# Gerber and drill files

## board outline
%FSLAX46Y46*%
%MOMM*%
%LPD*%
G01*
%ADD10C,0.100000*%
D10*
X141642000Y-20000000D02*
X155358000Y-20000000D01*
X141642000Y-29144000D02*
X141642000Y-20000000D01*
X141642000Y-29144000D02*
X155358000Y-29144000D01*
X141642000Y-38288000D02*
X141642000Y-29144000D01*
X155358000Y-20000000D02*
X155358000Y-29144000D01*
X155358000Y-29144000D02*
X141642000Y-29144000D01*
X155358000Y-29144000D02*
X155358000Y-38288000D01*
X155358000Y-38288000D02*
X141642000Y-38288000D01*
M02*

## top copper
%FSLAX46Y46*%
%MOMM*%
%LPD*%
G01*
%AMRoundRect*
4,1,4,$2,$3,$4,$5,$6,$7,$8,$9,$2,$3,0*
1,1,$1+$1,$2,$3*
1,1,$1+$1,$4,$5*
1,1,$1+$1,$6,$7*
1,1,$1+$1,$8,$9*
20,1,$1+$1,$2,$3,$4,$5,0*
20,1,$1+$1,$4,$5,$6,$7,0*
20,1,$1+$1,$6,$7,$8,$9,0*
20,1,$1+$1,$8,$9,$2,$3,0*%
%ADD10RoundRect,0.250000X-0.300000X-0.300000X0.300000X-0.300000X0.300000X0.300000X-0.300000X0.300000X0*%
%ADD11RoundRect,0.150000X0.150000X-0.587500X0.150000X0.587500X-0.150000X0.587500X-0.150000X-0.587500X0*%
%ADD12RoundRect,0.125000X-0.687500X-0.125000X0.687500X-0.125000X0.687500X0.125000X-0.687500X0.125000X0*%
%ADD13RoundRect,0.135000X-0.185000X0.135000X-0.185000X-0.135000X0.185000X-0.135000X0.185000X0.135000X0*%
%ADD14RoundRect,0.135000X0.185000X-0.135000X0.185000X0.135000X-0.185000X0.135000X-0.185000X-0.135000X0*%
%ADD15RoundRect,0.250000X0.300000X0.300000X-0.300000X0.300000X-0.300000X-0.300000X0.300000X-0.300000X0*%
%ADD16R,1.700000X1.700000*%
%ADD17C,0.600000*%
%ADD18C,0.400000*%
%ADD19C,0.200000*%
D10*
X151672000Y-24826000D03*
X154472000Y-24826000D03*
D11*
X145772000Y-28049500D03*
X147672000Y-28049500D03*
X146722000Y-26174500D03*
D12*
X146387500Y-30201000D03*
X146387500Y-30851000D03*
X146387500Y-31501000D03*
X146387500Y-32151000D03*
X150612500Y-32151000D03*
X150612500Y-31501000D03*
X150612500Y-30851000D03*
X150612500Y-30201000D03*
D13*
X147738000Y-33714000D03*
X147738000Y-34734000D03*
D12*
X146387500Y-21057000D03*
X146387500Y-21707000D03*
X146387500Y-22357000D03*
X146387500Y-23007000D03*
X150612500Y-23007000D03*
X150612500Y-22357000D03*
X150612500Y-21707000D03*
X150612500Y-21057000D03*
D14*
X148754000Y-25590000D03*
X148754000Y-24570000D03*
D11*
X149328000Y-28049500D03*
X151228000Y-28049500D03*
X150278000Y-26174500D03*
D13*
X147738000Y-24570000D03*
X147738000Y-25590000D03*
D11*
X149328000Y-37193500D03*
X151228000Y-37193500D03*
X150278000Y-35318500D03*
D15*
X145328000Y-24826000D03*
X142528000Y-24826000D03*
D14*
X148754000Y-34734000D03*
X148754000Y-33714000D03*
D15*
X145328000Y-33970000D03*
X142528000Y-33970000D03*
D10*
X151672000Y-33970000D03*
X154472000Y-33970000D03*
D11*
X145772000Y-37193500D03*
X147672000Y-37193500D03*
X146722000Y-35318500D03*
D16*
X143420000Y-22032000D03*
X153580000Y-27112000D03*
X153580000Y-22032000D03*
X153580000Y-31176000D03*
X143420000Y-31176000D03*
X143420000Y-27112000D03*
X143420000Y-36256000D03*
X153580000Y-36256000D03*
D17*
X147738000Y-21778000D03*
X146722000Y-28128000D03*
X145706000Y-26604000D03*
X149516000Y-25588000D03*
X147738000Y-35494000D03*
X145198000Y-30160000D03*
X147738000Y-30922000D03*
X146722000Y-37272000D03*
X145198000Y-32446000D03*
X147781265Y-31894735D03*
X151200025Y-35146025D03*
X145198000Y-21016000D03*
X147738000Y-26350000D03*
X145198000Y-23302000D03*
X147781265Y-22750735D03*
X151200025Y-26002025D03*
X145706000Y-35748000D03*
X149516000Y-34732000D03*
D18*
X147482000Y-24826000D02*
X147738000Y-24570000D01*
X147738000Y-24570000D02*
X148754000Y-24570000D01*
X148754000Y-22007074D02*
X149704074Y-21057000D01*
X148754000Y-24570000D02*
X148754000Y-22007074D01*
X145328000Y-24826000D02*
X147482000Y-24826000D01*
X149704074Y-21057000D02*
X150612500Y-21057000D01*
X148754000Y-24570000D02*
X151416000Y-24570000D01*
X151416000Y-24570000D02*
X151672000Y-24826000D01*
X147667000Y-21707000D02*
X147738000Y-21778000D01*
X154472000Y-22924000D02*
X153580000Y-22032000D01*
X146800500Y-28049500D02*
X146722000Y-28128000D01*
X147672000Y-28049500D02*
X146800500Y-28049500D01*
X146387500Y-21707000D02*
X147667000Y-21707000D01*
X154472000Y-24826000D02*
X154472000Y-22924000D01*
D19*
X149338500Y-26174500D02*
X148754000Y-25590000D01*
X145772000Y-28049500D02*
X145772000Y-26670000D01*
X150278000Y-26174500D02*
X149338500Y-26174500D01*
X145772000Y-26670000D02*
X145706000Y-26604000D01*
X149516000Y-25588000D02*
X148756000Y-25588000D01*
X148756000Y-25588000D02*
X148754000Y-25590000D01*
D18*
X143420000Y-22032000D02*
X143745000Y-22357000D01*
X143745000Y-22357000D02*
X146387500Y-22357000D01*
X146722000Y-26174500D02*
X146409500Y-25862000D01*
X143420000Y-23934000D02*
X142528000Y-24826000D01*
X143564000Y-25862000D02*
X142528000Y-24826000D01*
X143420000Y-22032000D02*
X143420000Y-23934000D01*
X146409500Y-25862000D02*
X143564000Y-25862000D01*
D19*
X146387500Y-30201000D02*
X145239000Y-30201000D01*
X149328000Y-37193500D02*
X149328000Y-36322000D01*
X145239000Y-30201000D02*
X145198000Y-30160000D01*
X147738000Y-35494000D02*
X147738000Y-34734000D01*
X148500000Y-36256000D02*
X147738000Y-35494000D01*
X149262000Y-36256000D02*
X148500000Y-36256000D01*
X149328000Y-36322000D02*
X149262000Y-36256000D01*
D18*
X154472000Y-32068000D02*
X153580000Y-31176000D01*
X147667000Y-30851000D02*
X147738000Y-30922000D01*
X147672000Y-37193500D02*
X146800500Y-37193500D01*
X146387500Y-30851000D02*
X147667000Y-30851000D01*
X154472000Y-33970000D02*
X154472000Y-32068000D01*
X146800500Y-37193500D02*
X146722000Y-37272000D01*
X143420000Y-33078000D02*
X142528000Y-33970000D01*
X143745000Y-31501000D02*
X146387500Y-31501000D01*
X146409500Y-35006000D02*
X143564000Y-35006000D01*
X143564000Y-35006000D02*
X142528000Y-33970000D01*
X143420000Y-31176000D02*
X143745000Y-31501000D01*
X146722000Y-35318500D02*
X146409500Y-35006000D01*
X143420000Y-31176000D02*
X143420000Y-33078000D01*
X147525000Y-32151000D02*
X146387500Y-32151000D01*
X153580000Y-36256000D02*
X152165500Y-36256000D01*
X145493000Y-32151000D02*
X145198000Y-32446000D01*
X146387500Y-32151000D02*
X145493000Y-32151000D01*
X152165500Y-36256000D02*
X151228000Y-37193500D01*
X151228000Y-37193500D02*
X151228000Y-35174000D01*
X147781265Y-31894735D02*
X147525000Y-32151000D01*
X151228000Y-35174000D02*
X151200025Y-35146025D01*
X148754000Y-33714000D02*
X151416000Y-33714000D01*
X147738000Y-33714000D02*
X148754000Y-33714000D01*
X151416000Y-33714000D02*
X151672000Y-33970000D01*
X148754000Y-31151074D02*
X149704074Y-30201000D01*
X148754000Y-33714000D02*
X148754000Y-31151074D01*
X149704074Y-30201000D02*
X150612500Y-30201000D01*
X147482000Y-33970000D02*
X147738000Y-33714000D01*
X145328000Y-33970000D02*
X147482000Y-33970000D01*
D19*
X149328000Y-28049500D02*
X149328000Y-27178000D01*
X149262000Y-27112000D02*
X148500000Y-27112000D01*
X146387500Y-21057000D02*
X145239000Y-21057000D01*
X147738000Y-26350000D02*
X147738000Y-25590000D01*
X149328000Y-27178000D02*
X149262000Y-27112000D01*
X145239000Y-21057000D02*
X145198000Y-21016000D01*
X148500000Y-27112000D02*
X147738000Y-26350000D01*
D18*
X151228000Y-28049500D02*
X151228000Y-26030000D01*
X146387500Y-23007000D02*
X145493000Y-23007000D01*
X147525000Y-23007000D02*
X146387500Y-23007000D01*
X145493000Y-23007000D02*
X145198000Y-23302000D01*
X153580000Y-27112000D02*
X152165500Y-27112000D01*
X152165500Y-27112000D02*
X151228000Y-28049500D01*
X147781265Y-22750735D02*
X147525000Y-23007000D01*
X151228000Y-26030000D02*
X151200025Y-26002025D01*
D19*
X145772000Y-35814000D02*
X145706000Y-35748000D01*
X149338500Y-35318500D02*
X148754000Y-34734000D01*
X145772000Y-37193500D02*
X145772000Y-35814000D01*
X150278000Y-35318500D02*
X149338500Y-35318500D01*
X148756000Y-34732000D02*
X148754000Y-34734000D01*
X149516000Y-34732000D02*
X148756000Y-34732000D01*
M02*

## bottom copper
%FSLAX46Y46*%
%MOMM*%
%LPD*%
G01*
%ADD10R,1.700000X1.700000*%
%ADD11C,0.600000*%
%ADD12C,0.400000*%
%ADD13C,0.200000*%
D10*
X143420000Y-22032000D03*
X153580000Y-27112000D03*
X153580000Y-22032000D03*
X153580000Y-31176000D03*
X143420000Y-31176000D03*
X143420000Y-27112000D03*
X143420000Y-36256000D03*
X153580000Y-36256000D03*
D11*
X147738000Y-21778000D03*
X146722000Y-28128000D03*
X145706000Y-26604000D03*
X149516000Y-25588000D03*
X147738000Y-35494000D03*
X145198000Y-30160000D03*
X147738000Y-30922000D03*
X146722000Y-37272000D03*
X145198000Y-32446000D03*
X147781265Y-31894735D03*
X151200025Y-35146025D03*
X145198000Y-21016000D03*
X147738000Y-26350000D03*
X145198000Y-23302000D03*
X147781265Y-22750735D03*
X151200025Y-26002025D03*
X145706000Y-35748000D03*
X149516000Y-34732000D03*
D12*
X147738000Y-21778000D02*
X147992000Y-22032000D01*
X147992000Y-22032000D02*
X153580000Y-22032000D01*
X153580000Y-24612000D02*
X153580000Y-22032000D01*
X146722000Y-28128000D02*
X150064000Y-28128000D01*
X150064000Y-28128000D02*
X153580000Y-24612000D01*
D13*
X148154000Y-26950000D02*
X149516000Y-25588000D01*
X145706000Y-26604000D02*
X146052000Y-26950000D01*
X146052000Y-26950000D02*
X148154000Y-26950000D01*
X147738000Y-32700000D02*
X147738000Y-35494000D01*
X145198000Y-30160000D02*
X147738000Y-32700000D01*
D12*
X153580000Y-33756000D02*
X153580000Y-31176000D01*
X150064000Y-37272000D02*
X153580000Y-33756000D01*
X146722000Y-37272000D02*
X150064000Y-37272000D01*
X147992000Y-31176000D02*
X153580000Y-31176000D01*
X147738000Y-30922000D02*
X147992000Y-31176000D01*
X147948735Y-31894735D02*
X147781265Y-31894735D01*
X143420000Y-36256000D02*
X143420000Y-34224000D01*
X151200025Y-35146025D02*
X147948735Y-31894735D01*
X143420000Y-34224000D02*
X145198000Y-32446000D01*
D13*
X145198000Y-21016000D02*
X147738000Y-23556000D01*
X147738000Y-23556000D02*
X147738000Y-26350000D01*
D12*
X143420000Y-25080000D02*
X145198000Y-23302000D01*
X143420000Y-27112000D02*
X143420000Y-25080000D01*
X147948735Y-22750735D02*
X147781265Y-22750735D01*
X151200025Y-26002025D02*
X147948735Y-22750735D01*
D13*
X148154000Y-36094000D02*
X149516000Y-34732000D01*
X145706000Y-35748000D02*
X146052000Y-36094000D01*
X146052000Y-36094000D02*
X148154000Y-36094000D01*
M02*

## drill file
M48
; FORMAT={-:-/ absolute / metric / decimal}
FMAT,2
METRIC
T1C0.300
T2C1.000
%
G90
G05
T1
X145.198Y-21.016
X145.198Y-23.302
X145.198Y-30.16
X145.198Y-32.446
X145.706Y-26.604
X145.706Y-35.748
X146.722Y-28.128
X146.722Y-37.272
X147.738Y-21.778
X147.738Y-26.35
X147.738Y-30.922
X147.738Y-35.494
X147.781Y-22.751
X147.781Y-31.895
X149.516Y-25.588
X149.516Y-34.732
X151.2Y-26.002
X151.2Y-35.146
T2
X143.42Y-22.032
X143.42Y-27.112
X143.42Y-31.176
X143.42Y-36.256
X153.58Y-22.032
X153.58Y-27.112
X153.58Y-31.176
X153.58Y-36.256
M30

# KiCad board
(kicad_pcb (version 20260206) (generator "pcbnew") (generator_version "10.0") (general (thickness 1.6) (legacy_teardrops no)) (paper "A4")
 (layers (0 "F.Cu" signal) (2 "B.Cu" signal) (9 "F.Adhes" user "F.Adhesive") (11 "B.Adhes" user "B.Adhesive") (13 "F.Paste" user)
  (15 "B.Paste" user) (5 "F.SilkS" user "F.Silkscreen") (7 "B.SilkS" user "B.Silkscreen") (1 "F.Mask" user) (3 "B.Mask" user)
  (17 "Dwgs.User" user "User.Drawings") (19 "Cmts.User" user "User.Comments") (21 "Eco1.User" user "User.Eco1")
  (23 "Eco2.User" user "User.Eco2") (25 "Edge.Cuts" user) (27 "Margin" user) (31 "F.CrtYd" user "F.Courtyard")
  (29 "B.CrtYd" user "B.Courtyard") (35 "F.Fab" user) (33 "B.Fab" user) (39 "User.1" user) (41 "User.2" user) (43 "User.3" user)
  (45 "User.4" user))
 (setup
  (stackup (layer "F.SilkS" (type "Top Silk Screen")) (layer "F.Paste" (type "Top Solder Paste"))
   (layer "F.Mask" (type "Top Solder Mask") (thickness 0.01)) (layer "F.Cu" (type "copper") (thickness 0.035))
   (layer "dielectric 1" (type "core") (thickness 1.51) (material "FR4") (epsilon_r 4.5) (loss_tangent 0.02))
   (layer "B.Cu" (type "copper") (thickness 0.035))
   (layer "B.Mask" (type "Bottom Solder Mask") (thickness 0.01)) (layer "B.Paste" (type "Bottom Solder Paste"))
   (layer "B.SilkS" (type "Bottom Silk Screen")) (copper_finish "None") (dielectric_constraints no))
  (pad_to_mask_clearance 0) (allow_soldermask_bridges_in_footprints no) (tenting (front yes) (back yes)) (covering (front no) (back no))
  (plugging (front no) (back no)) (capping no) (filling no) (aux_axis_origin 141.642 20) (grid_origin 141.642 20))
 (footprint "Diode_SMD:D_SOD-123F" (layer "F.Cu") (at 153.072 24.826)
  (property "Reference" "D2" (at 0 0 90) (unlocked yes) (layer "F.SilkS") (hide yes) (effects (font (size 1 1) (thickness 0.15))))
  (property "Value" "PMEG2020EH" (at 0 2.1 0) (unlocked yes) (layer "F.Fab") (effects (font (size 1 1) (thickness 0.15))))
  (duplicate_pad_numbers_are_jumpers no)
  (pad "1" smd roundrect (at -1.4 0) (size 1.1 1.1) (layers "F.Cu" "F.Mask" "F.Paste") (roundrect_rratio 0.2272727273) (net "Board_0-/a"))
  (pad "2" smd roundrect (at 1.4 0) (size 1.1 1.1) (layers "F.Cu" "F.Mask" "F.Paste") (roundrect_rratio 0.2272727273) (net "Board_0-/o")))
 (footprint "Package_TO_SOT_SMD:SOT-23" (layer "F.Cu") (at 146.722 27.112 90)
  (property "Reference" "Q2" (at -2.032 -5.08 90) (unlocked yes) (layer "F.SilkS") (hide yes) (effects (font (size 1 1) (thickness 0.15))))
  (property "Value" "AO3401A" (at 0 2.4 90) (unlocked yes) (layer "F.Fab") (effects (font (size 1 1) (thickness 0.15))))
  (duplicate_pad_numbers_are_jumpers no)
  (pad "1" smd roundrect (at -0.9375 -0.95 90) (size 1.475 0.6) (layers "F.Cu" "F.Mask" "F.Paste") (roundrect_rratio 0.25)
   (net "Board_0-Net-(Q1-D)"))
  (pad "2" smd roundrect (at -0.9375 0.95 90) (size 1.475 0.6) (layers "F.Cu" "F.Mask" "F.Paste") (roundrect_rratio 0.25) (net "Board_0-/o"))
  (pad "3" smd roundrect (at 0.9375 0 90) (size 1.475 0.6) (layers "F.Cu" "F.Mask" "F.Paste") (roundrect_rratio 0.25) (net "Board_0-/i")))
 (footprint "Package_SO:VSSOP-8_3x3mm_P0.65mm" (layer "F.Cu") (at 148.5 31.176)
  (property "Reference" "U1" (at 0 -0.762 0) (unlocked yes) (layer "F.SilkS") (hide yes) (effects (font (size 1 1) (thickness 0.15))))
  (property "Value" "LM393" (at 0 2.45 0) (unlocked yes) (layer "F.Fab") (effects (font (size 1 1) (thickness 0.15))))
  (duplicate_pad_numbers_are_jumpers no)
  (pad "1" smd roundrect (at -2.1125 -0.975) (size 1.625 0.5) (layers "F.Cu" "F.Mask" "F.Paste") (roundrect_rratio 0.25)
   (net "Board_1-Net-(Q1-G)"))
  (pad "2" smd roundrect (at -2.1125 -0.325) (size 1.625 0.5) (layers "F.Cu" "F.Mask" "F.Paste") (roundrect_rratio 0.25) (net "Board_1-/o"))
  (pad "3" smd roundrect (at -2.1125 0.325) (size 1.625 0.5) (layers "F.Cu" "F.Mask" "F.Paste") (roundrect_rratio 0.25) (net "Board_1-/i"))
  (pad "4" smd roundrect (at -2.1125 0.975) (size 1.625 0.5) (layers "F.Cu" "F.Mask" "F.Paste") (roundrect_rratio 0.25) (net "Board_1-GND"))
  (pad "5" smd roundrect (at 2.1125 0.975) (size 1.625 0.5) (layers "F.Cu" "F.Mask" "F.Paste") (roundrect_rratio 0.25)
   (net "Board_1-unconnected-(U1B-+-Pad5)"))
  (pad "6" smd roundrect (at 2.1125 0.325) (size 1.625 0.5) (layers "F.Cu" "F.Mask" "F.Paste") (roundrect_rratio 0.25)
   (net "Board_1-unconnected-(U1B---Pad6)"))
  (pad "7" smd roundrect (at 2.1125 -0.325) (size 1.625 0.5) (layers "F.Cu" "F.Mask" "F.Paste") (roundrect_rratio 0.25)
   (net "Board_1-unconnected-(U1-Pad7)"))
  (pad "8" smd roundrect (at 2.1125 -0.975) (size 1.625 0.5) (layers "F.Cu" "F.Mask" "F.Paste") (roundrect_rratio 0.25) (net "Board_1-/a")))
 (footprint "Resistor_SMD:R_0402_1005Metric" (layer "F.Cu") (at 147.738 34.224 -90)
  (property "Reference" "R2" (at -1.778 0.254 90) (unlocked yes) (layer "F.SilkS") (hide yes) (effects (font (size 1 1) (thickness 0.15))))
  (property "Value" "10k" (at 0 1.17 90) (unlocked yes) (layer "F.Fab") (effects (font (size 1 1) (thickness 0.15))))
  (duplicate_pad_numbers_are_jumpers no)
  (pad "1" smd roundrect (at -0.51 0 270) (size 0.54 0.64) (layers "F.Cu" "F.Mask" "F.Paste") (roundrect_rratio 0.25) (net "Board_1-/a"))
  (pad "2" smd roundrect (at 0.51 0 270) (size 0.54 0.64) (layers "F.Cu" "F.Mask" "F.Paste") (roundrect_rratio 0.25)
   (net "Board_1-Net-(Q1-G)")))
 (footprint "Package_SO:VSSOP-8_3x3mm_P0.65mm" (layer "F.Cu") (at 148.5 22.032)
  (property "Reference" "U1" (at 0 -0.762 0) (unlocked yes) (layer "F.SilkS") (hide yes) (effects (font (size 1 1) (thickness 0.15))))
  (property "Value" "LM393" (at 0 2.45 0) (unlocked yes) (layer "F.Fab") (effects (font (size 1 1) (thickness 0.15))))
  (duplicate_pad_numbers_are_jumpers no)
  (pad "1" smd roundrect (at -2.1125 -0.975) (size 1.625 0.5) (layers "F.Cu" "F.Mask" "F.Paste") (roundrect_rratio 0.25)
   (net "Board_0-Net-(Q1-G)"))
  (pad "2" smd roundrect (at -2.1125 -0.325) (size 1.625 0.5) (layers "F.Cu" "F.Mask" "F.Paste") (roundrect_rratio 0.25) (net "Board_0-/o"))
  (pad "3" smd roundrect (at -2.1125 0.325) (size 1.625 0.5) (layers "F.Cu" "F.Mask" "F.Paste") (roundrect_rratio 0.25) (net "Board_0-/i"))
  (pad "4" smd roundrect (at -2.1125 0.975) (size 1.625 0.5) (layers "F.Cu" "F.Mask" "F.Paste") (roundrect_rratio 0.25) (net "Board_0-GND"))
  (pad "5" smd roundrect (at 2.1125 0.975) (size 1.625 0.5) (layers "F.Cu" "F.Mask" "F.Paste") (roundrect_rratio 0.25)
   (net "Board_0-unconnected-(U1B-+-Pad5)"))
  (pad "6" smd roundrect (at 2.1125 0.325) (size 1.625 0.5) (layers "F.Cu" "F.Mask" "F.Paste") (roundrect_rratio 0.25)
   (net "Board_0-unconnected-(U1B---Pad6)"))
  (pad "7" smd roundrect (at 2.1125 -0.325) (size 1.625 0.5) (layers "F.Cu" "F.Mask" "F.Paste") (roundrect_rratio 0.25)
   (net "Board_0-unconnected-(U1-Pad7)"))
  (pad "8" smd roundrect (at 2.1125 -0.975) (size 1.625 0.5) (layers "F.Cu" "F.Mask" "F.Paste") (roundrect_rratio 0.25) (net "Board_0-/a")))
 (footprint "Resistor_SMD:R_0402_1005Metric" (layer "F.Cu") (at 148.754 25.08 90)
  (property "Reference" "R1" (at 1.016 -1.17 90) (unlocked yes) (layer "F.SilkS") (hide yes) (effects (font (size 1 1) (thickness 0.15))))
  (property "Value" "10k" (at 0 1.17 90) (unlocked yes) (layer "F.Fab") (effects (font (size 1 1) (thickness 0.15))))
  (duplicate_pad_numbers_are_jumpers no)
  (pad "1" smd roundrect (at -0.51 0 90) (size 0.54 0.64) (layers "F.Cu" "F.Mask" "F.Paste") (roundrect_rratio 0.25)
   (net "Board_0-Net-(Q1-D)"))
  (pad "2" smd roundrect (at 0.51 0 90) (size 0.54 0.64) (layers "F.Cu" "F.Mask" "F.Paste") (roundrect_rratio 0.25) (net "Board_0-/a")))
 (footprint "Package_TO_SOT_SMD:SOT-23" (layer "F.Cu") (at 150.278 27.112 90)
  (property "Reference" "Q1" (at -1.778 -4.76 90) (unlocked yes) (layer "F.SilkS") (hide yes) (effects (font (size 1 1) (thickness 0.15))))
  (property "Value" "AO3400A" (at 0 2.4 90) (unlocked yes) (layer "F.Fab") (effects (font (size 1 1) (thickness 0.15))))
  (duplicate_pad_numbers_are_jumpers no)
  (pad "1" smd roundrect (at -0.9375 -0.95 90) (size 1.475 0.6) (layers "F.Cu" "F.Mask" "F.Paste") (roundrect_rratio 0.25)
   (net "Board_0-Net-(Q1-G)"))
  (pad "2" smd roundrect (at -0.9375 0.95 90) (size 1.475 0.6) (layers "F.Cu" "F.Mask" "F.Paste") (roundrect_rratio 0.25)
   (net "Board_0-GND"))
  (pad "3" smd roundrect (at 0.9375 0 90) (size 1.475 0.6) (layers "F.Cu" "F.Mask" "F.Paste") (roundrect_rratio 0.25)
   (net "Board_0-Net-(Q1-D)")))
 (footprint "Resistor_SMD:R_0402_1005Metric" (layer "F.Cu") (at 147.738 25.08 -90)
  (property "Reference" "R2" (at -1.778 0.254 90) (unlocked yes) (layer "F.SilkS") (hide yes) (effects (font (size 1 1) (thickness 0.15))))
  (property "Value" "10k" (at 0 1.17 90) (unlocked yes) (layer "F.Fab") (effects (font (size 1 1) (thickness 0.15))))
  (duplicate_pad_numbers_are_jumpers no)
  (pad "1" smd roundrect (at -0.51 0 270) (size 0.54 0.64) (layers "F.Cu" "F.Mask" "F.Paste") (roundrect_rratio 0.25) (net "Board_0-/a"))
  (pad "2" smd roundrect (at 0.51 0 270) (size 0.54 0.64) (layers "F.Cu" "F.Mask" "F.Paste") (roundrect_rratio 0.25)
   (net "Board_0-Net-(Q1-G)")))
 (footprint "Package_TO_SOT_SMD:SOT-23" (layer "F.Cu") (at 150.278 36.256 90)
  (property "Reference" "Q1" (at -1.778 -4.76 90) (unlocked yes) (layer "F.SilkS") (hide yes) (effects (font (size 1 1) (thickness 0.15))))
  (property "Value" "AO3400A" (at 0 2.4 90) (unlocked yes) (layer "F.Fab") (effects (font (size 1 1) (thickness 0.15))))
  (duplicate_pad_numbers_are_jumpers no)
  (pad "1" smd roundrect (at -0.9375 -0.95 90) (size 1.475 0.6) (layers "F.Cu" "F.Mask" "F.Paste") (roundrect_rratio 0.25)
   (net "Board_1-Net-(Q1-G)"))
  (pad "2" smd roundrect (at -0.9375 0.95 90) (size 1.475 0.6) (layers "F.Cu" "F.Mask" "F.Paste") (roundrect_rratio 0.25)
   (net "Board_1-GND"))
  (pad "3" smd roundrect (at 0.9375 0 90) (size 1.475 0.6) (layers "F.Cu" "F.Mask" "F.Paste") (roundrect_rratio 0.25)
   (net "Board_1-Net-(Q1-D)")))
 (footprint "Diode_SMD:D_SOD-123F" (layer "F.Cu") (at 143.928 24.826 180)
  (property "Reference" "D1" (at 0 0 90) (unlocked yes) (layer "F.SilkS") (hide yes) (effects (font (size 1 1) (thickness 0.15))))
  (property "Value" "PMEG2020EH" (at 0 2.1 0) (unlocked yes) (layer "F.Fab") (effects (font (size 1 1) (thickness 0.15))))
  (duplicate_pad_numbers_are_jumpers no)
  (pad "1" smd roundrect (at -1.4 0 180) (size 1.1 1.1) (layers "F.Cu" "F.Mask" "F.Paste") (roundrect_rratio 0.2272727273)
   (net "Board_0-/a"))
  (pad "2" smd roundrect (at 1.4 0 180) (size 1.1 1.1) (layers "F.Cu" "F.Mask" "F.Paste") (roundrect_rratio 0.2272727273) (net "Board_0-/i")))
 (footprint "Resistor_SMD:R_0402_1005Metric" (layer "F.Cu") (at 148.754 34.224 90)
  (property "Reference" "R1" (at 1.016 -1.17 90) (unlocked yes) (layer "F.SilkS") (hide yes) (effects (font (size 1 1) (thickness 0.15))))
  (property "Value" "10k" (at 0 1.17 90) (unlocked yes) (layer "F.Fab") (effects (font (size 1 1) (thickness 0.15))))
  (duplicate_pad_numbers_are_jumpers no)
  (pad "1" smd roundrect (at -0.51 0 90) (size 0.54 0.64) (layers "F.Cu" "F.Mask" "F.Paste") (roundrect_rratio 0.25)
   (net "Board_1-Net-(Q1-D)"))
  (pad "2" smd roundrect (at 0.51 0 90) (size 0.54 0.64) (layers "F.Cu" "F.Mask" "F.Paste") (roundrect_rratio 0.25) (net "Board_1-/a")))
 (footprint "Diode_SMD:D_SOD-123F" (layer "F.Cu") (at 143.928 33.97 180)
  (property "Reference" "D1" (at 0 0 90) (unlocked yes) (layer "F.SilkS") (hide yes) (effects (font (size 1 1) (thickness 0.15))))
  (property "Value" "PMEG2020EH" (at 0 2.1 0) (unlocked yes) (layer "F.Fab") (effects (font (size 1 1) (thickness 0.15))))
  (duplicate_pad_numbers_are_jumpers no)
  (pad "1" smd roundrect (at -1.4 0 180) (size 1.1 1.1) (layers "F.Cu" "F.Mask" "F.Paste") (roundrect_rratio 0.2272727273)
   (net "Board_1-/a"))
  (pad "2" smd roundrect (at 1.4 0 180) (size 1.1 1.1) (layers "F.Cu" "F.Mask" "F.Paste") (roundrect_rratio 0.2272727273) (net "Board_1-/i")))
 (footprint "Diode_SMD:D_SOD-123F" (layer "F.Cu") (at 153.072 33.97)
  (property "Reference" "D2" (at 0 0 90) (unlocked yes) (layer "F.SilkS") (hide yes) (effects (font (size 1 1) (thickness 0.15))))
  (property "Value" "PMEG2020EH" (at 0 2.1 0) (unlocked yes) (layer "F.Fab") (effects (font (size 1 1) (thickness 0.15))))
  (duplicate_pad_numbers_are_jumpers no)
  (pad "1" smd roundrect (at -1.4 0) (size 1.1 1.1) (layers "F.Cu" "F.Mask" "F.Paste") (roundrect_rratio 0.2272727273) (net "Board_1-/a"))
  (pad "2" smd roundrect (at 1.4 0) (size 1.1 1.1) (layers "F.Cu" "F.Mask" "F.Paste") (roundrect_rratio 0.2272727273) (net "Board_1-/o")))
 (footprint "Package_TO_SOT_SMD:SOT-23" (layer "F.Cu") (at 146.722 36.256 90)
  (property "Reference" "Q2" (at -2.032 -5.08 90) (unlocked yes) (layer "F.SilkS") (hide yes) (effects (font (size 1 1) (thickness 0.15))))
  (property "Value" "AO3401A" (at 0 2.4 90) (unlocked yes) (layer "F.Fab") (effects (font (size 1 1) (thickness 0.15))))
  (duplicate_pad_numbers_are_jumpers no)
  (pad "1" smd roundrect (at -0.9375 -0.95 90) (size 1.475 0.6) (layers "F.Cu" "F.Mask" "F.Paste") (roundrect_rratio 0.25)
   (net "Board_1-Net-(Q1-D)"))
  (pad "2" smd roundrect (at -0.9375 0.95 90) (size 1.475 0.6) (layers "F.Cu" "F.Mask" "F.Paste") (roundrect_rratio 0.25) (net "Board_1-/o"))
  (pad "3" smd roundrect (at 0.9375 0 90) (size 1.475 0.6) (layers "F.Cu" "F.Mask" "F.Paste") (roundrect_rratio 0.25) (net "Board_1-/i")))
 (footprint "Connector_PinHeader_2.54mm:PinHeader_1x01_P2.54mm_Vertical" (layer "B.Cu") (at 143.42 22.032 180)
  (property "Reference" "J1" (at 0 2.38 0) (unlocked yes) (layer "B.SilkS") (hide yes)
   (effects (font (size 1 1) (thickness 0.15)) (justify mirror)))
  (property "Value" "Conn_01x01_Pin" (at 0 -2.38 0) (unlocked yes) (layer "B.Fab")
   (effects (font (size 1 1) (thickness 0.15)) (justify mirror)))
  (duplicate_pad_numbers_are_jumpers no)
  (pad "1" thru_hole rect (at 0 0 180) (size 1.7 1.7) (drill 1) (layers "*.Cu" "*.Mask") (remove_unused_layers no) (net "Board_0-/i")))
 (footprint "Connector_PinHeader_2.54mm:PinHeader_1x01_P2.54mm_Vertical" (layer "B.Cu") (at 153.58 27.112 180)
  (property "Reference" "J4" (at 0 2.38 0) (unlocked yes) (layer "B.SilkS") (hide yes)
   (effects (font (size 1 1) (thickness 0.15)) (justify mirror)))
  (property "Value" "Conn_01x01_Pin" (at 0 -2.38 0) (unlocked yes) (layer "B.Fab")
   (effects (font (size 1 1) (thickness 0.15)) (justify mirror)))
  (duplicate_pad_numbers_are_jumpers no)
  (pad "1" thru_hole rect (at 0 0 180) (size 1.7 1.7) (drill 1) (layers "*.Cu" "*.Mask") (remove_unused_layers no) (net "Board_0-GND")))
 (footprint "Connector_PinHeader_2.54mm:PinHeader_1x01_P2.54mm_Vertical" (layer "B.Cu") (at 153.58 22.032 180)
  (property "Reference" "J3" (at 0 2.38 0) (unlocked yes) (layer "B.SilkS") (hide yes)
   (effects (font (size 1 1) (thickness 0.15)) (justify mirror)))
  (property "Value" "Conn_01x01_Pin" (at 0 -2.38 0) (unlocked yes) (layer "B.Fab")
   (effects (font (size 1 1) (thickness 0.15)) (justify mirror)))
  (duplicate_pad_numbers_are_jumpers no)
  (pad "1" thru_hole rect (at 0 0 180) (size 1.7 1.7) (drill 1) (layers "*.Cu" "*.Mask") (remove_unused_layers no) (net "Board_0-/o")))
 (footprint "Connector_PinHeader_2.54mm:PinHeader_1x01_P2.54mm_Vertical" (layer "B.Cu") (at 153.58 31.176 180)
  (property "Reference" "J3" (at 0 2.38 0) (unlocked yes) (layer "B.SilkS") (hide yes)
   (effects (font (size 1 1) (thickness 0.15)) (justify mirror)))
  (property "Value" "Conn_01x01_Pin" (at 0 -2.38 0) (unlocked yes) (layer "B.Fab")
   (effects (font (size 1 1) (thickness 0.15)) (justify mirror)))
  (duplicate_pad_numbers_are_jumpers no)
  (pad "1" thru_hole rect (at 0 0 180) (size 1.7 1.7) (drill 1) (layers "*.Cu" "*.Mask") (remove_unused_layers no) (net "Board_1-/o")))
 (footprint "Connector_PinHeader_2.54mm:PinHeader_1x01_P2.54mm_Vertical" (layer "B.Cu") (at 143.42 31.176 180)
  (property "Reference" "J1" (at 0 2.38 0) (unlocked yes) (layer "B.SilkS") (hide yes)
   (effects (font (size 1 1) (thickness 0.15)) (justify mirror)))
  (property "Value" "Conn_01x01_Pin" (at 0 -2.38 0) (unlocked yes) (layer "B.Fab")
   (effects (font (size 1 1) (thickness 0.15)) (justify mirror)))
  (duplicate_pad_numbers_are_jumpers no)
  (pad "1" thru_hole rect (at 0 0 180) (size 1.7 1.7) (drill 1) (layers "*.Cu" "*.Mask") (remove_unused_layers no) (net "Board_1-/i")))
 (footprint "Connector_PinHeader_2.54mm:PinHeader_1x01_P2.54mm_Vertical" (layer "B.Cu") (at 143.42 27.112 180)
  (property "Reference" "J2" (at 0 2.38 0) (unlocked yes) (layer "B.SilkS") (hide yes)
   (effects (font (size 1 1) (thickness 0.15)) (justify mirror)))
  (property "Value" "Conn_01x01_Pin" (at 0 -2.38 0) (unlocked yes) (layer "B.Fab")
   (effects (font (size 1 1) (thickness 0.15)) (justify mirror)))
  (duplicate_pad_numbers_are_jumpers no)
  (pad "1" thru_hole rect (at 0 0 180) (size 1.7 1.7) (drill 1) (layers "*.Cu" "*.Mask") (remove_unused_layers no) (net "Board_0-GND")))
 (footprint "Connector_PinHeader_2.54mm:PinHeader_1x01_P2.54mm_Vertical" (layer "B.Cu") (at 143.42 36.256 180)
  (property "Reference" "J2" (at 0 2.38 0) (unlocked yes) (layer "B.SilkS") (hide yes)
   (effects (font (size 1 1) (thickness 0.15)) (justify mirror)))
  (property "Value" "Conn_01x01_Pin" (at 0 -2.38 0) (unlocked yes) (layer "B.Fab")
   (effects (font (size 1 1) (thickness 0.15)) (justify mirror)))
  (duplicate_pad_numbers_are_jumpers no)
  (pad "1" thru_hole rect (at 0 0 180) (size 1.7 1.7) (drill 1) (layers "*.Cu" "*.Mask") (remove_unused_layers no) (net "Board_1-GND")))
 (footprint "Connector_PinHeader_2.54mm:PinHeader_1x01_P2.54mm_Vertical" (layer "B.Cu") (at 153.58 36.256 180)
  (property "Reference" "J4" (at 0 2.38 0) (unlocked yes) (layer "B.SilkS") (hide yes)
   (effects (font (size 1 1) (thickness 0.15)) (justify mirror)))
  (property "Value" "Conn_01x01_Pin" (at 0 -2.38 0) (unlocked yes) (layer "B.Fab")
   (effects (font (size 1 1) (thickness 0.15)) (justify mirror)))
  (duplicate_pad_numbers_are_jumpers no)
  (pad "1" thru_hole rect (at 0 0 180) (size 1.7 1.7) (drill 1) (layers "*.Cu" "*.Mask") (remove_unused_layers no) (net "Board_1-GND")))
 (gr_line (start 141.642 20) (end 155.358 20) (stroke (width 0.1) (type default)) (layer "Edge.Cuts"))
 (gr_line (start 141.642 29.144) (end 141.642 20) (stroke (width 0.1) (type default)) (layer "Edge.Cuts"))
 (gr_line (start 141.642 29.144) (end 155.358 29.144) (stroke (width 0.1) (type default)) (layer "Edge.Cuts"))
 (gr_line (start 141.642 38.288) (end 141.642 29.144) (stroke (width 0.1) (type default)) (layer "Edge.Cuts"))
 (gr_line (start 155.358 20) (end 155.358 29.144) (stroke (width 0.1) (type default)) (layer "Edge.Cuts"))
 (gr_line (start 155.358 29.144) (end 141.642 29.144) (stroke (width 0.1) (type default)) (layer "Edge.Cuts"))
 (gr_line (start 155.358 29.144) (end 155.358 38.288) (stroke (width 0.1) (type default)) (layer "Edge.Cuts"))
 (gr_line (start 155.358 38.288) (end 141.642 38.288) (stroke (width 0.1) (type default)) (layer "Edge.Cuts"))
 (segment (start 147.482 24.826) (end 147.738 24.57) (width 0.4) (layer "F.Cu") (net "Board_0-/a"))
 (segment (start 147.738 24.57) (end 148.754 24.57) (width 0.4) (layer "F.Cu") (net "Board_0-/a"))
 (segment (start 148.754 22.007074) (end 149.704074 21.057) (width 0.4) (layer "F.Cu") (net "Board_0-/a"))
 (segment (start 148.754 24.57) (end 148.754 22.007074) (width 0.4) (layer "F.Cu") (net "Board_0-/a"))
 (segment (start 145.328 24.826) (end 147.482 24.826) (width 0.4) (layer "F.Cu") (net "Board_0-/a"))
 (segment (start 149.704074 21.057) (end 150.6125 21.057) (width 0.4) (layer "F.Cu") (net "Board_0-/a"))
 (segment (start 148.754 24.57) (end 151.416 24.57) (width 0.4) (layer "F.Cu") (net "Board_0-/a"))
 (segment (start 151.416 24.57) (end 151.672 24.826) (width 0.4) (layer "F.Cu") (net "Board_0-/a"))
 (segment (start 147.667 21.707) (end 147.738 21.778) (width 0.4) (layer "F.Cu") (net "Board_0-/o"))
 (segment (start 154.472 22.924) (end 153.58 22.032) (width 0.4) (layer "F.Cu") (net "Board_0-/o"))
 (segment (start 146.8005 28.0495) (end 146.722 28.128) (width 0.4) (layer "F.Cu") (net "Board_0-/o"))
 (segment (start 147.672 28.0495) (end 146.8005 28.0495) (width 0.4) (layer "F.Cu") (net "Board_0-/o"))
 (segment (start 146.3875 21.707) (end 147.667 21.707) (width 0.4) (layer "F.Cu") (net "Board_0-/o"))
 (segment (start 154.472 24.826) (end 154.472 22.924) (width 0.4) (layer "F.Cu") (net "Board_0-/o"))
 (via (at 147.738 21.778) (size 0.6) (drill 0.3) (layers "F.Cu" "B.Cu") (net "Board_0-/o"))
 (via (at 146.722 28.128) (size 0.6) (drill 0.3) (layers "F.Cu" "B.Cu") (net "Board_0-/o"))
 (segment (start 147.738 21.778) (end 147.992 22.032) (width 0.4) (layer "B.Cu") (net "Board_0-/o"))
 (segment (start 147.992 22.032) (end 153.58 22.032) (width 0.4) (layer "B.Cu") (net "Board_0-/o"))
 (segment (start 153.58 24.612) (end 153.58 22.032) (width 0.4) (layer "B.Cu") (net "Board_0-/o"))
 (segment (start 146.722 28.128) (end 150.064 28.128) (width 0.4) (layer "B.Cu") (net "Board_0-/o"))
 (segment (start 150.064 28.128) (end 153.58 24.612) (width 0.4) (layer "B.Cu") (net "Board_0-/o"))
 (segment (start 149.3385 26.1745) (end 148.754 25.59) (width 0.2) (layer "F.Cu") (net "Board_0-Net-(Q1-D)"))
 (segment (start 145.772 28.0495) (end 145.772 26.67) (width 0.2) (layer "F.Cu") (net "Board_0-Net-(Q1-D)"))
 (segment (start 150.278 26.1745) (end 149.3385 26.1745) (width 0.2) (layer "F.Cu") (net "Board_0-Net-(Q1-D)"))
 (segment (start 145.772 26.67) (end 145.706 26.604) (width 0.2) (layer "F.Cu") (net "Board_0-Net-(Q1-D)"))
 (segment (start 149.516 25.588) (end 148.756 25.588) (width 0.2) (layer "F.Cu") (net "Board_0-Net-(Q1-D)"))
 (segment (start 148.756 25.588) (end 148.754 25.59) (width 0.2) (layer "F.Cu") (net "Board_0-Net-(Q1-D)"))
 (via (at 145.706 26.604) (size 0.6) (drill 0.3) (layers "F.Cu" "B.Cu") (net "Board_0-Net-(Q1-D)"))
 (via (at 149.516 25.588) (size 0.6) (drill 0.3) (layers "F.Cu" "B.Cu") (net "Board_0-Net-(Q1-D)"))
 (segment (start 148.154 26.95) (end 149.516 25.588) (width 0.2) (layer "B.Cu") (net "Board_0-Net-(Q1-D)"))
 (segment (start 145.706 26.604) (end 146.052 26.95) (width 0.2) (layer "B.Cu") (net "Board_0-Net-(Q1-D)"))
 (segment (start 146.052 26.95) (end 148.154 26.95) (width 0.2) (layer "B.Cu") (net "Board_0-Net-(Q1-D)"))
 (segment (start 143.42 22.032) (end 143.745 22.357) (width 0.4) (layer "F.Cu") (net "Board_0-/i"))
 (segment (start 143.745 22.357) (end 146.3875 22.357) (width 0.4) (layer "F.Cu") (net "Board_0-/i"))
 (segment (start 146.722 26.1745) (end 146.4095 25.862) (width 0.4) (layer "F.Cu") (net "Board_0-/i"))
 (segment (start 143.42 23.934) (end 142.528 24.826) (width 0.4) (layer "F.Cu") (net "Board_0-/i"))
 (segment (start 143.564 25.862) (end 142.528 24.826) (width 0.4) (layer "F.Cu") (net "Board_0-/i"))
 (segment (start 143.42 22.032) (end 143.42 23.934) (width 0.4) (layer "F.Cu") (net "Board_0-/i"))
 (segment (start 146.4095 25.862) (end 143.564 25.862) (width 0.4) (layer "F.Cu") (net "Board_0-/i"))
 (segment (start 146.3875 30.201) (end 145.239 30.201) (width 0.2) (layer "F.Cu") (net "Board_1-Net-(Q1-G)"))
 (segment (start 149.328 37.1935) (end 149.328 36.322) (width 0.2) (layer "F.Cu") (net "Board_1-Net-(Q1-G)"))
 (segment (start 145.239 30.201) (end 145.198 30.16) (width 0.2) (layer "F.Cu") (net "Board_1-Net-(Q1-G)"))
 (segment (start 147.738 35.494) (end 147.738 34.734) (width 0.2) (layer "F.Cu") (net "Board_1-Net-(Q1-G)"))
 (segment (start 148.5 36.256) (end 147.738 35.494) (width 0.2) (layer "F.Cu") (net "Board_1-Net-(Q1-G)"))
 (segment (start 149.262 36.256) (end 148.5 36.256) (width 0.2) (layer "F.Cu") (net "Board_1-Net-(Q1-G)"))
 (segment (start 149.328 36.322) (end 149.262 36.256) (width 0.2) (layer "F.Cu") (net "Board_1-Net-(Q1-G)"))
 (via (at 147.738 35.494) (size 0.6) (drill 0.3) (layers "F.Cu" "B.Cu") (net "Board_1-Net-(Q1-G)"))
 (via (at 145.198 30.16) (size 0.6) (drill 0.3) (layers "F.Cu" "B.Cu") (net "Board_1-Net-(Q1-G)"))
 (segment (start 147.738 32.7) (end 147.738 35.494) (width 0.2) (layer "B.Cu") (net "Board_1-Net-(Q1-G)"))
 (segment (start 145.198 30.16) (end 147.738 32.7) (width 0.2) (layer "B.Cu") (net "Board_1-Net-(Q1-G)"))
 (segment (start 154.472 32.068) (end 153.58 31.176) (width 0.4) (layer "F.Cu") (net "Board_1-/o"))
 (segment (start 147.667 30.851) (end 147.738 30.922) (width 0.4) (layer "F.Cu") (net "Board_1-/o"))
 (segment (start 147.672 37.1935) (end 146.8005 37.1935) (width 0.4) (layer "F.Cu") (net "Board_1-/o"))
 (segment (start 146.3875 30.851) (end 147.667 30.851) (width 0.4) (layer "F.Cu") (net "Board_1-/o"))
 (segment (start 154.472 33.97) (end 154.472 32.068) (width 0.4) (layer "F.Cu") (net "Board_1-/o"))
 (segment (start 146.8005 37.1935) (end 146.722 37.272) (width 0.4) (layer "F.Cu") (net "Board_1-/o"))
 (via (at 147.738 30.922) (size 0.6) (drill 0.3) (layers "F.Cu" "B.Cu") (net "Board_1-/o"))
 (via (at 146.722 37.272) (size 0.6) (drill 0.3) (layers "F.Cu" "B.Cu") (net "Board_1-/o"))
 (segment (start 153.58 33.756) (end 153.58 31.176) (width 0.4) (layer "B.Cu") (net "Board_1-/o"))
 (segment (start 150.064 37.272) (end 153.58 33.756) (width 0.4) (layer "B.Cu") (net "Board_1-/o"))
 (segment (start 146.722 37.272) (end 150.064 37.272) (width 0.4) (layer "B.Cu") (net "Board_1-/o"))
 (segment (start 147.992 31.176) (end 153.58 31.176) (width 0.4) (layer "B.Cu") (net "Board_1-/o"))
 (segment (start 147.738 30.922) (end 147.992 31.176) (width 0.4) (layer "B.Cu") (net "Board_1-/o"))
 (segment (start 143.42 33.078) (end 142.528 33.97) (width 0.4) (layer "F.Cu") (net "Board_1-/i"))
 (segment (start 143.745 31.501) (end 146.3875 31.501) (width 0.4) (layer "F.Cu") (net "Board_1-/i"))
 (segment (start 146.4095 35.006) (end 143.564 35.006) (width 0.4) (layer "F.Cu") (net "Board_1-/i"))
 (segment (start 143.564 35.006) (end 142.528 33.97) (width 0.4) (layer "F.Cu") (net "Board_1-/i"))
 (segment (start 143.42 31.176) (end 143.745 31.501) (width 0.4) (layer "F.Cu") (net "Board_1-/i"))
 (segment (start 146.722 35.3185) (end 146.4095 35.006) (width 0.4) (layer "F.Cu") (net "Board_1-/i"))
 (segment (start 143.42 31.176) (end 143.42 33.078) (width 0.4) (layer "F.Cu") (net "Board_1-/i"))
 (segment (start 147.525 32.151) (end 146.3875 32.151) (width 0.4) (layer "F.Cu") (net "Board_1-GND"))
 (segment (start 153.58 36.256) (end 152.1655 36.256) (width 0.4) (layer "F.Cu") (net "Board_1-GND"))
 (segment (start 145.493 32.151) (end 145.198 32.446) (width 0.4) (layer "F.Cu") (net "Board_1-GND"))
 (segment (start 146.3875 32.151) (end 145.493 32.151) (width 0.4) (layer "F.Cu") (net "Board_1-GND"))
 (segment (start 152.1655 36.256) (end 151.228 37.1935) (width 0.4) (layer "F.Cu") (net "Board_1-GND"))
 (segment (start 151.228 37.1935) (end 151.228 35.174) (width 0.4) (layer "F.Cu") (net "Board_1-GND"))
 (segment (start 147.781265 31.894735) (end 147.525 32.151) (width 0.4) (layer "F.Cu") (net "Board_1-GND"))
 (segment (start 151.228 35.174) (end 151.200025 35.146025) (width 0.4) (layer "F.Cu") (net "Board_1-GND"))
 (via blind (at 145.198 32.446) (size 0.6) (drill 0.3) (layers "F.Cu" "B.Cu") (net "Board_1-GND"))
 (via (at 147.781265 31.894735) (size 0.6) (drill 0.3) (layers "F.Cu" "B.Cu") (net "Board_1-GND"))
 (via (at 151.200025 35.146025) (size 0.6) (drill 0.3) (layers "F.Cu" "B.Cu") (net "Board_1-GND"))
 (segment (start 147.948735 31.894735) (end 147.781265 31.894735) (width 0.4) (layer "B.Cu") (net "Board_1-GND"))
 (segment (start 143.42 36.256) (end 143.42 34.224) (width 0.4) (layer "B.Cu") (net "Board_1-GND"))
 (segment (start 151.200025 35.146025) (end 147.948735 31.894735) (width 0.4) (layer "B.Cu") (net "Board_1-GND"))
 (segment (start 143.42 34.224) (end 145.198 32.446) (width 0.4) (layer "B.Cu") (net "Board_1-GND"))
 (segment (start 148.754 33.714) (end 151.416 33.714) (width 0.4) (layer "F.Cu") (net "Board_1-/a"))
 (segment (start 147.738 33.714) (end 148.754 33.714) (width 0.4) (layer "F.Cu") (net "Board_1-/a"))
 (segment (start 151.416 33.714) (end 151.672 33.97) (width 0.4) (layer "F.Cu") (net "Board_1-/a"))
 (segment (start 148.754 31.151074) (end 149.704074 30.201) (width 0.4) (layer "F.Cu") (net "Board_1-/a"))
 (segment (start 148.754 33.714) (end 148.754 31.151074) (width 0.4) (layer "F.Cu") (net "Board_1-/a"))
 (segment (start 149.704074 30.201) (end 150.6125 30.201) (width 0.4) (layer "F.Cu") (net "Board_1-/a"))
 (segment (start 147.482 33.97) (end 147.738 33.714) (width 0.4) (layer "F.Cu") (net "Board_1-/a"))
 (segment (start 145.328 33.97) (end 147.482 33.97) (width 0.4) (layer "F.Cu") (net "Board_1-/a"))
 (segment (start 149.328 28.0495) (end 149.328 27.178) (width 0.2) (layer "F.Cu") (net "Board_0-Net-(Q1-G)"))
 (segment (start 149.262 27.112) (end 148.5 27.112) (width 0.2) (layer "F.Cu") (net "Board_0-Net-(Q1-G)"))
 (segment (start 146.3875 21.057) (end 145.239 21.057) (width 0.2) (layer "F.Cu") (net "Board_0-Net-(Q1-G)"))
 (segment (start 147.738 26.35) (end 147.738 25.59) (width 0.2) (layer "F.Cu") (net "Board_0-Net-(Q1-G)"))
 (segment (start 149.328 27.178) (end 149.262 27.112) (width 0.2) (layer "F.Cu") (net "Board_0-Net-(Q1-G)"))
 (segment (start 145.239 21.057) (end 145.198 21.016) (width 0.2) (layer "F.Cu") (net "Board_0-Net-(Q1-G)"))
 (segment (start 148.5 27.112) (end 147.738 26.35) (width 0.2) (layer "F.Cu") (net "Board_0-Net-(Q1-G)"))
 (via (at 145.198 21.016) (size 0.6) (drill 0.3) (layers "F.Cu" "B.Cu") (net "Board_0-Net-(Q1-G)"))
 (via (at 147.738 26.35) (size 0.6) (drill 0.3) (layers "F.Cu" "B.Cu") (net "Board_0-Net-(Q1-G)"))
 (segment (start 145.198 21.016) (end 147.738 23.556) (width 0.2) (layer "B.Cu") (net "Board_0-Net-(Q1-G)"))
 (segment (start 147.738 23.556) (end 147.738 26.35) (width 0.2) (layer "B.Cu") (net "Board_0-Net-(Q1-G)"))
 (segment (start 151.228 28.0495) (end 151.228 26.03) (width 0.4) (layer "F.Cu") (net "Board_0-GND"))
 (segment (start 146.3875 23.007) (end 145.493 23.007) (width 0.4) (layer "F.Cu") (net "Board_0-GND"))
 (segment (start 147.525 23.007) (end 146.3875 23.007) (width 0.4) (layer "F.Cu") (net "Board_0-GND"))
 (segment (start 145.493 23.007) (end 145.198 23.302) (width 0.4) (layer "F.Cu") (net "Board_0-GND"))
 (segment (start 153.58 27.112) (end 152.1655 27.112) (width 0.4) (layer "F.Cu") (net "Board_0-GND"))
 (segment (start 152.1655 27.112) (end 151.228 28.0495) (width 0.4) (layer "F.Cu") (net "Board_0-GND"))
 (segment (start 147.781265 22.750735) (end 147.525 23.007) (width 0.4) (layer "F.Cu") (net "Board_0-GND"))
 (segment (start 151.228 26.03) (end 151.200025 26.002025) (width 0.4) (layer "F.Cu") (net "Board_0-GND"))
 (via blind (at 145.198 23.302) (size 0.6) (drill 0.3) (layers "F.Cu" "B.Cu") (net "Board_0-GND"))
 (via (at 147.781265 22.750735) (size 0.6) (drill 0.3) (layers "F.Cu" "B.Cu") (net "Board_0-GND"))
 (via (at 151.200025 26.002025) (size 0.6) (drill 0.3) (layers "F.Cu" "B.Cu") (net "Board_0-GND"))
 (segment (start 143.42 25.08) (end 145.198 23.302) (width 0.4) (layer "B.Cu") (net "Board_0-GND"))
 (segment (start 143.42 27.112) (end 143.42 25.08) (width 0.4) (layer "B.Cu") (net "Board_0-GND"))
 (segment (start 147.948735 22.750735) (end 147.781265 22.750735) (width 0.4) (layer "B.Cu") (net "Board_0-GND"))
 (segment (start 151.200025 26.002025) (end 147.948735 22.750735) (width 0.4) (layer "B.Cu") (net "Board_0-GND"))
 (segment (start 145.772 35.814) (end 145.706 35.748) (width 0.2) (layer "F.Cu") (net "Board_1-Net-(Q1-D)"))
 (segment (start 149.3385 35.3185) (end 148.754 34.734) (width 0.2) (layer "F.Cu") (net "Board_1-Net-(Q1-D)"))
 (segment (start 145.772 37.1935) (end 145.772 35.814) (width 0.2) (layer "F.Cu") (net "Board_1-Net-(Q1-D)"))
 (segment (start 150.278 35.3185) (end 149.3385 35.3185) (width 0.2) (layer "F.Cu") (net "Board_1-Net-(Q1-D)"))
 (segment (start 148.756 34.732) (end 148.754 34.734) (width 0.2) (layer "F.Cu") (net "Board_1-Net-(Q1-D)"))
 (segment (start 149.516 34.732) (end 148.756 34.732) (width 0.2) (layer "F.Cu") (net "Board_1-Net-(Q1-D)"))
 (via (at 145.706 35.748) (size 0.6) (drill 0.3) (layers "F.Cu" "B.Cu") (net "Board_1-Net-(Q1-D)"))
 (via (at 149.516 34.732) (size 0.6) (drill 0.3) (layers "F.Cu" "B.Cu") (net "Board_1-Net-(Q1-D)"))
 (segment (start 148.154 36.094) (end 149.516 34.732) (width 0.2) (layer "B.Cu") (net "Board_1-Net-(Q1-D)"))
 (segment (start 145.706 35.748) (end 146.052 36.094) (width 0.2) (layer "B.Cu") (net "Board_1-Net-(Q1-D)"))
 (segment (start 146.052 36.094) (end 148.154 36.094) (width 0.2) (layer "B.Cu") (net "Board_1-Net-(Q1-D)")))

